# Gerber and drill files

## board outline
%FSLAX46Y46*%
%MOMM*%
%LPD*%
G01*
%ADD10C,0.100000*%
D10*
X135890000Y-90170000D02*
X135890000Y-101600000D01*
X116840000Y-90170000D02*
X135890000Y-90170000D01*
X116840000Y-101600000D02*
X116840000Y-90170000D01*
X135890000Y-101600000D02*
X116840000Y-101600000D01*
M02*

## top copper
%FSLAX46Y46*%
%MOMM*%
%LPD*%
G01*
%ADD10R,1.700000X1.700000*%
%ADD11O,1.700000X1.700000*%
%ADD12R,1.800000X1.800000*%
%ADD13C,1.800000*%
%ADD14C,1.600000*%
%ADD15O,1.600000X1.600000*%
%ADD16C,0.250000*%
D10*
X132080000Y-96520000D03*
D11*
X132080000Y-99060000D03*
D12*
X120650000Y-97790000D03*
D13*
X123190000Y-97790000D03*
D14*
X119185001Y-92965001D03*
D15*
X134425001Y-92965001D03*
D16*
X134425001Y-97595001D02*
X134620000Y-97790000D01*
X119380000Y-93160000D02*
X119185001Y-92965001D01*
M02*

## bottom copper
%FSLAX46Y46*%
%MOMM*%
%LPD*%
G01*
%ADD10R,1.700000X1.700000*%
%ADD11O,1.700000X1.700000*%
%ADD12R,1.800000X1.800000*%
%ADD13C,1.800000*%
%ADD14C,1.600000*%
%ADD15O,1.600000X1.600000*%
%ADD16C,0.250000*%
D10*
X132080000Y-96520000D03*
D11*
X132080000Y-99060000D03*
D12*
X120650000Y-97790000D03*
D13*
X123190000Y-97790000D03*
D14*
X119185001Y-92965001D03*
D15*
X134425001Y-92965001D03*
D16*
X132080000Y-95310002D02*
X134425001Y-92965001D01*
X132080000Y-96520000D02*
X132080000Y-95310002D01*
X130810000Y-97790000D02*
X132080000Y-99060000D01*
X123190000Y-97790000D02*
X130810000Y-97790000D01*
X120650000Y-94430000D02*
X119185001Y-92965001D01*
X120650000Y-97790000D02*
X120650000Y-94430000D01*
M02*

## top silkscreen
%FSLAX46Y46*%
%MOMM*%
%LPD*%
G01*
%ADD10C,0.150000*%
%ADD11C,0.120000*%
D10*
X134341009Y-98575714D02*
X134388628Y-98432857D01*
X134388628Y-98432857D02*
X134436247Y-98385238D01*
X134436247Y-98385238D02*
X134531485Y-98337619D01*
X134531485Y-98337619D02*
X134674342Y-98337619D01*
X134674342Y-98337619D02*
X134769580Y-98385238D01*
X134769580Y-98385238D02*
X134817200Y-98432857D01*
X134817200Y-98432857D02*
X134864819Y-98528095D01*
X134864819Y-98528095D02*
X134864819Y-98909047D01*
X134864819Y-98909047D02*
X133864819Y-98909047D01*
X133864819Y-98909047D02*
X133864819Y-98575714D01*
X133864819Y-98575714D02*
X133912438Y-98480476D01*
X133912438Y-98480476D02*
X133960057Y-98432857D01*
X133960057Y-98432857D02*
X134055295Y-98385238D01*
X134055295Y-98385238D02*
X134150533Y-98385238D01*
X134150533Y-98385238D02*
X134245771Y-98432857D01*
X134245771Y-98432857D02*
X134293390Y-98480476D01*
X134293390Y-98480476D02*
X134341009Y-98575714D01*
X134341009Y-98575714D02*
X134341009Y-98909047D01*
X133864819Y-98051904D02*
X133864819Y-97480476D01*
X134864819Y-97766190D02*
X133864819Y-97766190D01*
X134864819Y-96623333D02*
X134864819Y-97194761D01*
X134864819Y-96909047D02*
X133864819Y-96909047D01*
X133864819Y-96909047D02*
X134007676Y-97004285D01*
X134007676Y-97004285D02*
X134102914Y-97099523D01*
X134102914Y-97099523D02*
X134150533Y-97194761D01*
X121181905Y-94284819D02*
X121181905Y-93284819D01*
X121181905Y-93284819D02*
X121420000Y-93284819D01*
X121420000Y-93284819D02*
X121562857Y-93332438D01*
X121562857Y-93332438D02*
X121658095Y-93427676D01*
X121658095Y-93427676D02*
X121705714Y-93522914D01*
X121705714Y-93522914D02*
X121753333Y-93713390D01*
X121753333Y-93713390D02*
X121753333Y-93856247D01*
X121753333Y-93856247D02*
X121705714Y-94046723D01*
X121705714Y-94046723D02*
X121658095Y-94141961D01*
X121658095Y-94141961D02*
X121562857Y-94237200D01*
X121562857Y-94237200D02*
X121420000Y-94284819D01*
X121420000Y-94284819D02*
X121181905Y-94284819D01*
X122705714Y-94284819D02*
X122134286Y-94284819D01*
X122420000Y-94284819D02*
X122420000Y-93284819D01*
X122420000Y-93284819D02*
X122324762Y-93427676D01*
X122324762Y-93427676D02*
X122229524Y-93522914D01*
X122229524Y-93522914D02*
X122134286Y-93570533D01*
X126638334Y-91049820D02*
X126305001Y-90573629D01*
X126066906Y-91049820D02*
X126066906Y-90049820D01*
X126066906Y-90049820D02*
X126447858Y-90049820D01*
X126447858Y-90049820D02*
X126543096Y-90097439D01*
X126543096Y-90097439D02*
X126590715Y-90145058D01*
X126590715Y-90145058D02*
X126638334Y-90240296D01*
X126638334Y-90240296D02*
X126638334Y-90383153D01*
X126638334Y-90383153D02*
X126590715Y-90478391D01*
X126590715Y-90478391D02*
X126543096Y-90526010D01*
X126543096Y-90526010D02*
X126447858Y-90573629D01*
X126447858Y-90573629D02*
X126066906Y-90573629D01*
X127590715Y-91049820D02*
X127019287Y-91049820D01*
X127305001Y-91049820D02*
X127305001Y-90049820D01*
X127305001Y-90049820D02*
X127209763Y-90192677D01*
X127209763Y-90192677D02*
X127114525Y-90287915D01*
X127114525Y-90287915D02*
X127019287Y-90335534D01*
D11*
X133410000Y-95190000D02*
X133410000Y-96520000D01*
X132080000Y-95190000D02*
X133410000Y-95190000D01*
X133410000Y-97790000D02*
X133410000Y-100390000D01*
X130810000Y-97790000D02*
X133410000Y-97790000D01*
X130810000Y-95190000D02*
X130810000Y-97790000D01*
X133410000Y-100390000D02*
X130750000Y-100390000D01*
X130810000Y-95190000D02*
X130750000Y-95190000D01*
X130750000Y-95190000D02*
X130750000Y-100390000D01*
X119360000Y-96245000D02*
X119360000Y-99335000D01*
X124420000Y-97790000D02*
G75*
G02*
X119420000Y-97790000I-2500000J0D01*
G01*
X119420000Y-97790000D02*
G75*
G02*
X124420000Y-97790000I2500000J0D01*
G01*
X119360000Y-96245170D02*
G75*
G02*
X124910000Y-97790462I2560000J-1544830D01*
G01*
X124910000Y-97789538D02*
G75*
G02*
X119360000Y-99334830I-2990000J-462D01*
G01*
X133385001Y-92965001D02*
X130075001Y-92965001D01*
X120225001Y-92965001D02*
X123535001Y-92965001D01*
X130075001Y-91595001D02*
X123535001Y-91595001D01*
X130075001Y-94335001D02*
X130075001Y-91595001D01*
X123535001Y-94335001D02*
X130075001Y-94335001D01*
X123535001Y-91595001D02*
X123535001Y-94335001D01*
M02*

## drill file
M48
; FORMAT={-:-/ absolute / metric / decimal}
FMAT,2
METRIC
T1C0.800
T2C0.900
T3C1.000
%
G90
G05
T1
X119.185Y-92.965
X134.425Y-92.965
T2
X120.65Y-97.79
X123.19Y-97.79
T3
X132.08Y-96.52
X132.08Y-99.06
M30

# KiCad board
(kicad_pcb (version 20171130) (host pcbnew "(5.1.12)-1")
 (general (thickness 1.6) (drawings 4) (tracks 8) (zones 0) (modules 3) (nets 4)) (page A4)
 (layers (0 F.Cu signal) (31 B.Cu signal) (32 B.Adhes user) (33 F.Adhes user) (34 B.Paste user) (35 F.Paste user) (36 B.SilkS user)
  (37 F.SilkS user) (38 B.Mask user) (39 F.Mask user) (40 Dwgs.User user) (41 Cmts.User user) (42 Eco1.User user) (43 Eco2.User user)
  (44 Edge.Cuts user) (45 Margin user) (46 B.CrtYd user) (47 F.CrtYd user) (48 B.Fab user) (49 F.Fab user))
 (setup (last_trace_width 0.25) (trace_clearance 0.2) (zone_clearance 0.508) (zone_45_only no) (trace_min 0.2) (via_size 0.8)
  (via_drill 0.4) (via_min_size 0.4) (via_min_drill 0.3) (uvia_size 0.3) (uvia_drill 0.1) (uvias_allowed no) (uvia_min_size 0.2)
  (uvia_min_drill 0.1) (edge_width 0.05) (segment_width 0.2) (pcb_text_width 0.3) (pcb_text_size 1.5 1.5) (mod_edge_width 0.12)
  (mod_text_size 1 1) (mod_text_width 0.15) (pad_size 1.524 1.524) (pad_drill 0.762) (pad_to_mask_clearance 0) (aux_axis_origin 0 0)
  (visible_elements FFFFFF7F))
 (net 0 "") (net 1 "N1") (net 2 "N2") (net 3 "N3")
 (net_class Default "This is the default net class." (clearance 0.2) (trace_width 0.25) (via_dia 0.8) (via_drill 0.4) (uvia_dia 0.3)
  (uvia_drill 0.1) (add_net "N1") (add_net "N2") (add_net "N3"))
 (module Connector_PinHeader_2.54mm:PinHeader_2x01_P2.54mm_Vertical (layer F.Cu) (at 132.08 96.52 270)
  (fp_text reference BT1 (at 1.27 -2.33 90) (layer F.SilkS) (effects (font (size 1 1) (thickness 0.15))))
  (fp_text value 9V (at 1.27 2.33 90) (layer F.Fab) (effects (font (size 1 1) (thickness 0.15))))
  (fp_line (start -1.33 -1.33) (end 0 -1.33) (layer F.SilkS) (width 0.12))
  (fp_line (start -1.33 0) (end -1.33 -1.33) (layer F.SilkS) (width 0.12))
  (fp_line (start 1.27 -1.33) (end 3.87 -1.33) (layer F.SilkS) (width 0.12))
  (fp_line (start 1.27 1.27) (end 1.27 -1.33) (layer F.SilkS) (width 0.12))
  (fp_line (start -1.33 1.27) (end 1.27 1.27) (layer F.SilkS) (width 0.12))
  (fp_line (start 3.87 -1.33) (end 3.87 1.33) (layer F.SilkS) (width 0.12))
  (fp_line (start -1.33 1.27) (end -1.33 1.33) (layer F.SilkS) (width 0.12))
  (fp_line (start -1.33 1.33) (end 3.87 1.33) (layer F.SilkS) (width 0.12))
  (pad 1 thru_hole rect (at 0 0 270) (size 1.7 1.7) (drill 1) (layers *.Cu *.Mask) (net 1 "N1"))
  (pad 2 thru_hole oval (at 2.54 0 270) (size 1.7 1.7) (drill 1) (layers *.Cu *.Mask) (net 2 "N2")))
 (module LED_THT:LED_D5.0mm (layer F.Cu) (at 120.65 97.79)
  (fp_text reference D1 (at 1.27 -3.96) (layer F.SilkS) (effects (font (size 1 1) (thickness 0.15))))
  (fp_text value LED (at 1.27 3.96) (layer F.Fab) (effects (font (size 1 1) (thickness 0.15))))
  (fp_line (start -1.29 -1.545) (end -1.29 1.545) (layer F.SilkS) (width 0.12))
  (fp_circle (center 1.27 0) (end 3.77 0) (layer F.SilkS) (width 0.12))
  (fp_arc (start 1.27 0) (end -1.29 -1.54483) (angle 148.9) (layer F.SilkS) (width 0.12))
  (fp_arc (start 1.27 0) (end -1.29 1.54483) (angle -148.9) (layer F.SilkS) (width 0.12))
  (pad 1 thru_hole rect (at 0 0) (size 1.8 1.8) (drill 0.9) (layers *.Cu *.Mask) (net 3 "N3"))
  (pad 2 thru_hole circle (at 2.54 0) (size 1.8 1.8) (drill 0.9) (layers *.Cu *.Mask) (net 2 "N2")))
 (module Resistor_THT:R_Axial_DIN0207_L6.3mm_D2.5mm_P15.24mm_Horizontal (layer F.Cu) (at 119.185001 92.965001)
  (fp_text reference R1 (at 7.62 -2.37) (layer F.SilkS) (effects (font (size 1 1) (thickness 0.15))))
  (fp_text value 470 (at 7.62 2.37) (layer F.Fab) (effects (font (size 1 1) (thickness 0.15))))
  (fp_line (start 14.2 0) (end 10.89 0) (layer F.SilkS) (width 0.12))
  (fp_line (start 1.04 0) (end 4.35 0) (layer F.SilkS) (width 0.12))
  (fp_line (start 10.89 -1.37) (end 4.35 -1.37) (layer F.SilkS) (width 0.12))
  (fp_line (start 10.89 1.37) (end 10.89 -1.37) (layer F.SilkS) (width 0.12))
  (fp_line (start 4.35 1.37) (end 10.89 1.37) (layer F.SilkS) (width 0.12))
  (fp_line (start 4.35 -1.37) (end 4.35 1.37) (layer F.SilkS) (width 0.12))
  (pad 1 thru_hole circle (at 0 0) (size 1.6 1.6) (drill 0.8) (layers *.Cu *.Mask) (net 3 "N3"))
  (pad 2 thru_hole oval (at 15.24 0) (size 1.6 1.6) (drill 0.8) (layers *.Cu *.Mask) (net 1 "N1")))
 (gr_line (start 135.89 90.17) (end 135.89 101.6) (layer Edge.Cuts) (width 0.1))
 (gr_line (start 116.84 90.17) (end 135.89 90.17) (layer Edge.Cuts) (width 0.1))
 (gr_line (start 116.84 101.6) (end 116.84 90.17) (layer Edge.Cuts) (width 0.1))
 (gr_line (start 135.89 101.6) (end 116.84 101.6) (layer Edge.Cuts) (width 0.1))
 (segment (start 134.425001 97.595001) (end 134.62 97.79) (width 0.25) (layer F.Cu) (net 1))
 (segment (start 132.08 95.310002) (end 134.425001 92.965001) (width 0.25) (layer B.Cu) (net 1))
 (segment (start 132.08 96.52) (end 132.08 95.310002) (width 0.25) (layer B.Cu) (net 1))
 (segment (start 130.81 97.79) (end 132.08 99.06) (width 0.25) (layer B.Cu) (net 2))
 (segment (start 123.19 97.79) (end 130.81 97.79) (width 0.25) (layer B.Cu) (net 2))
 (segment (start 119.38 93.16) (end 119.185001 92.965001) (width 0.25) (layer F.Cu) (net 3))
 (segment (start 120.65 94.43) (end 119.185001 92.965001) (width 0.25) (layer B.Cu) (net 3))
 (segment (start 120.65 97.79) (end 120.65 94.43) (width 0.25) (layer B.Cu) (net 3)))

